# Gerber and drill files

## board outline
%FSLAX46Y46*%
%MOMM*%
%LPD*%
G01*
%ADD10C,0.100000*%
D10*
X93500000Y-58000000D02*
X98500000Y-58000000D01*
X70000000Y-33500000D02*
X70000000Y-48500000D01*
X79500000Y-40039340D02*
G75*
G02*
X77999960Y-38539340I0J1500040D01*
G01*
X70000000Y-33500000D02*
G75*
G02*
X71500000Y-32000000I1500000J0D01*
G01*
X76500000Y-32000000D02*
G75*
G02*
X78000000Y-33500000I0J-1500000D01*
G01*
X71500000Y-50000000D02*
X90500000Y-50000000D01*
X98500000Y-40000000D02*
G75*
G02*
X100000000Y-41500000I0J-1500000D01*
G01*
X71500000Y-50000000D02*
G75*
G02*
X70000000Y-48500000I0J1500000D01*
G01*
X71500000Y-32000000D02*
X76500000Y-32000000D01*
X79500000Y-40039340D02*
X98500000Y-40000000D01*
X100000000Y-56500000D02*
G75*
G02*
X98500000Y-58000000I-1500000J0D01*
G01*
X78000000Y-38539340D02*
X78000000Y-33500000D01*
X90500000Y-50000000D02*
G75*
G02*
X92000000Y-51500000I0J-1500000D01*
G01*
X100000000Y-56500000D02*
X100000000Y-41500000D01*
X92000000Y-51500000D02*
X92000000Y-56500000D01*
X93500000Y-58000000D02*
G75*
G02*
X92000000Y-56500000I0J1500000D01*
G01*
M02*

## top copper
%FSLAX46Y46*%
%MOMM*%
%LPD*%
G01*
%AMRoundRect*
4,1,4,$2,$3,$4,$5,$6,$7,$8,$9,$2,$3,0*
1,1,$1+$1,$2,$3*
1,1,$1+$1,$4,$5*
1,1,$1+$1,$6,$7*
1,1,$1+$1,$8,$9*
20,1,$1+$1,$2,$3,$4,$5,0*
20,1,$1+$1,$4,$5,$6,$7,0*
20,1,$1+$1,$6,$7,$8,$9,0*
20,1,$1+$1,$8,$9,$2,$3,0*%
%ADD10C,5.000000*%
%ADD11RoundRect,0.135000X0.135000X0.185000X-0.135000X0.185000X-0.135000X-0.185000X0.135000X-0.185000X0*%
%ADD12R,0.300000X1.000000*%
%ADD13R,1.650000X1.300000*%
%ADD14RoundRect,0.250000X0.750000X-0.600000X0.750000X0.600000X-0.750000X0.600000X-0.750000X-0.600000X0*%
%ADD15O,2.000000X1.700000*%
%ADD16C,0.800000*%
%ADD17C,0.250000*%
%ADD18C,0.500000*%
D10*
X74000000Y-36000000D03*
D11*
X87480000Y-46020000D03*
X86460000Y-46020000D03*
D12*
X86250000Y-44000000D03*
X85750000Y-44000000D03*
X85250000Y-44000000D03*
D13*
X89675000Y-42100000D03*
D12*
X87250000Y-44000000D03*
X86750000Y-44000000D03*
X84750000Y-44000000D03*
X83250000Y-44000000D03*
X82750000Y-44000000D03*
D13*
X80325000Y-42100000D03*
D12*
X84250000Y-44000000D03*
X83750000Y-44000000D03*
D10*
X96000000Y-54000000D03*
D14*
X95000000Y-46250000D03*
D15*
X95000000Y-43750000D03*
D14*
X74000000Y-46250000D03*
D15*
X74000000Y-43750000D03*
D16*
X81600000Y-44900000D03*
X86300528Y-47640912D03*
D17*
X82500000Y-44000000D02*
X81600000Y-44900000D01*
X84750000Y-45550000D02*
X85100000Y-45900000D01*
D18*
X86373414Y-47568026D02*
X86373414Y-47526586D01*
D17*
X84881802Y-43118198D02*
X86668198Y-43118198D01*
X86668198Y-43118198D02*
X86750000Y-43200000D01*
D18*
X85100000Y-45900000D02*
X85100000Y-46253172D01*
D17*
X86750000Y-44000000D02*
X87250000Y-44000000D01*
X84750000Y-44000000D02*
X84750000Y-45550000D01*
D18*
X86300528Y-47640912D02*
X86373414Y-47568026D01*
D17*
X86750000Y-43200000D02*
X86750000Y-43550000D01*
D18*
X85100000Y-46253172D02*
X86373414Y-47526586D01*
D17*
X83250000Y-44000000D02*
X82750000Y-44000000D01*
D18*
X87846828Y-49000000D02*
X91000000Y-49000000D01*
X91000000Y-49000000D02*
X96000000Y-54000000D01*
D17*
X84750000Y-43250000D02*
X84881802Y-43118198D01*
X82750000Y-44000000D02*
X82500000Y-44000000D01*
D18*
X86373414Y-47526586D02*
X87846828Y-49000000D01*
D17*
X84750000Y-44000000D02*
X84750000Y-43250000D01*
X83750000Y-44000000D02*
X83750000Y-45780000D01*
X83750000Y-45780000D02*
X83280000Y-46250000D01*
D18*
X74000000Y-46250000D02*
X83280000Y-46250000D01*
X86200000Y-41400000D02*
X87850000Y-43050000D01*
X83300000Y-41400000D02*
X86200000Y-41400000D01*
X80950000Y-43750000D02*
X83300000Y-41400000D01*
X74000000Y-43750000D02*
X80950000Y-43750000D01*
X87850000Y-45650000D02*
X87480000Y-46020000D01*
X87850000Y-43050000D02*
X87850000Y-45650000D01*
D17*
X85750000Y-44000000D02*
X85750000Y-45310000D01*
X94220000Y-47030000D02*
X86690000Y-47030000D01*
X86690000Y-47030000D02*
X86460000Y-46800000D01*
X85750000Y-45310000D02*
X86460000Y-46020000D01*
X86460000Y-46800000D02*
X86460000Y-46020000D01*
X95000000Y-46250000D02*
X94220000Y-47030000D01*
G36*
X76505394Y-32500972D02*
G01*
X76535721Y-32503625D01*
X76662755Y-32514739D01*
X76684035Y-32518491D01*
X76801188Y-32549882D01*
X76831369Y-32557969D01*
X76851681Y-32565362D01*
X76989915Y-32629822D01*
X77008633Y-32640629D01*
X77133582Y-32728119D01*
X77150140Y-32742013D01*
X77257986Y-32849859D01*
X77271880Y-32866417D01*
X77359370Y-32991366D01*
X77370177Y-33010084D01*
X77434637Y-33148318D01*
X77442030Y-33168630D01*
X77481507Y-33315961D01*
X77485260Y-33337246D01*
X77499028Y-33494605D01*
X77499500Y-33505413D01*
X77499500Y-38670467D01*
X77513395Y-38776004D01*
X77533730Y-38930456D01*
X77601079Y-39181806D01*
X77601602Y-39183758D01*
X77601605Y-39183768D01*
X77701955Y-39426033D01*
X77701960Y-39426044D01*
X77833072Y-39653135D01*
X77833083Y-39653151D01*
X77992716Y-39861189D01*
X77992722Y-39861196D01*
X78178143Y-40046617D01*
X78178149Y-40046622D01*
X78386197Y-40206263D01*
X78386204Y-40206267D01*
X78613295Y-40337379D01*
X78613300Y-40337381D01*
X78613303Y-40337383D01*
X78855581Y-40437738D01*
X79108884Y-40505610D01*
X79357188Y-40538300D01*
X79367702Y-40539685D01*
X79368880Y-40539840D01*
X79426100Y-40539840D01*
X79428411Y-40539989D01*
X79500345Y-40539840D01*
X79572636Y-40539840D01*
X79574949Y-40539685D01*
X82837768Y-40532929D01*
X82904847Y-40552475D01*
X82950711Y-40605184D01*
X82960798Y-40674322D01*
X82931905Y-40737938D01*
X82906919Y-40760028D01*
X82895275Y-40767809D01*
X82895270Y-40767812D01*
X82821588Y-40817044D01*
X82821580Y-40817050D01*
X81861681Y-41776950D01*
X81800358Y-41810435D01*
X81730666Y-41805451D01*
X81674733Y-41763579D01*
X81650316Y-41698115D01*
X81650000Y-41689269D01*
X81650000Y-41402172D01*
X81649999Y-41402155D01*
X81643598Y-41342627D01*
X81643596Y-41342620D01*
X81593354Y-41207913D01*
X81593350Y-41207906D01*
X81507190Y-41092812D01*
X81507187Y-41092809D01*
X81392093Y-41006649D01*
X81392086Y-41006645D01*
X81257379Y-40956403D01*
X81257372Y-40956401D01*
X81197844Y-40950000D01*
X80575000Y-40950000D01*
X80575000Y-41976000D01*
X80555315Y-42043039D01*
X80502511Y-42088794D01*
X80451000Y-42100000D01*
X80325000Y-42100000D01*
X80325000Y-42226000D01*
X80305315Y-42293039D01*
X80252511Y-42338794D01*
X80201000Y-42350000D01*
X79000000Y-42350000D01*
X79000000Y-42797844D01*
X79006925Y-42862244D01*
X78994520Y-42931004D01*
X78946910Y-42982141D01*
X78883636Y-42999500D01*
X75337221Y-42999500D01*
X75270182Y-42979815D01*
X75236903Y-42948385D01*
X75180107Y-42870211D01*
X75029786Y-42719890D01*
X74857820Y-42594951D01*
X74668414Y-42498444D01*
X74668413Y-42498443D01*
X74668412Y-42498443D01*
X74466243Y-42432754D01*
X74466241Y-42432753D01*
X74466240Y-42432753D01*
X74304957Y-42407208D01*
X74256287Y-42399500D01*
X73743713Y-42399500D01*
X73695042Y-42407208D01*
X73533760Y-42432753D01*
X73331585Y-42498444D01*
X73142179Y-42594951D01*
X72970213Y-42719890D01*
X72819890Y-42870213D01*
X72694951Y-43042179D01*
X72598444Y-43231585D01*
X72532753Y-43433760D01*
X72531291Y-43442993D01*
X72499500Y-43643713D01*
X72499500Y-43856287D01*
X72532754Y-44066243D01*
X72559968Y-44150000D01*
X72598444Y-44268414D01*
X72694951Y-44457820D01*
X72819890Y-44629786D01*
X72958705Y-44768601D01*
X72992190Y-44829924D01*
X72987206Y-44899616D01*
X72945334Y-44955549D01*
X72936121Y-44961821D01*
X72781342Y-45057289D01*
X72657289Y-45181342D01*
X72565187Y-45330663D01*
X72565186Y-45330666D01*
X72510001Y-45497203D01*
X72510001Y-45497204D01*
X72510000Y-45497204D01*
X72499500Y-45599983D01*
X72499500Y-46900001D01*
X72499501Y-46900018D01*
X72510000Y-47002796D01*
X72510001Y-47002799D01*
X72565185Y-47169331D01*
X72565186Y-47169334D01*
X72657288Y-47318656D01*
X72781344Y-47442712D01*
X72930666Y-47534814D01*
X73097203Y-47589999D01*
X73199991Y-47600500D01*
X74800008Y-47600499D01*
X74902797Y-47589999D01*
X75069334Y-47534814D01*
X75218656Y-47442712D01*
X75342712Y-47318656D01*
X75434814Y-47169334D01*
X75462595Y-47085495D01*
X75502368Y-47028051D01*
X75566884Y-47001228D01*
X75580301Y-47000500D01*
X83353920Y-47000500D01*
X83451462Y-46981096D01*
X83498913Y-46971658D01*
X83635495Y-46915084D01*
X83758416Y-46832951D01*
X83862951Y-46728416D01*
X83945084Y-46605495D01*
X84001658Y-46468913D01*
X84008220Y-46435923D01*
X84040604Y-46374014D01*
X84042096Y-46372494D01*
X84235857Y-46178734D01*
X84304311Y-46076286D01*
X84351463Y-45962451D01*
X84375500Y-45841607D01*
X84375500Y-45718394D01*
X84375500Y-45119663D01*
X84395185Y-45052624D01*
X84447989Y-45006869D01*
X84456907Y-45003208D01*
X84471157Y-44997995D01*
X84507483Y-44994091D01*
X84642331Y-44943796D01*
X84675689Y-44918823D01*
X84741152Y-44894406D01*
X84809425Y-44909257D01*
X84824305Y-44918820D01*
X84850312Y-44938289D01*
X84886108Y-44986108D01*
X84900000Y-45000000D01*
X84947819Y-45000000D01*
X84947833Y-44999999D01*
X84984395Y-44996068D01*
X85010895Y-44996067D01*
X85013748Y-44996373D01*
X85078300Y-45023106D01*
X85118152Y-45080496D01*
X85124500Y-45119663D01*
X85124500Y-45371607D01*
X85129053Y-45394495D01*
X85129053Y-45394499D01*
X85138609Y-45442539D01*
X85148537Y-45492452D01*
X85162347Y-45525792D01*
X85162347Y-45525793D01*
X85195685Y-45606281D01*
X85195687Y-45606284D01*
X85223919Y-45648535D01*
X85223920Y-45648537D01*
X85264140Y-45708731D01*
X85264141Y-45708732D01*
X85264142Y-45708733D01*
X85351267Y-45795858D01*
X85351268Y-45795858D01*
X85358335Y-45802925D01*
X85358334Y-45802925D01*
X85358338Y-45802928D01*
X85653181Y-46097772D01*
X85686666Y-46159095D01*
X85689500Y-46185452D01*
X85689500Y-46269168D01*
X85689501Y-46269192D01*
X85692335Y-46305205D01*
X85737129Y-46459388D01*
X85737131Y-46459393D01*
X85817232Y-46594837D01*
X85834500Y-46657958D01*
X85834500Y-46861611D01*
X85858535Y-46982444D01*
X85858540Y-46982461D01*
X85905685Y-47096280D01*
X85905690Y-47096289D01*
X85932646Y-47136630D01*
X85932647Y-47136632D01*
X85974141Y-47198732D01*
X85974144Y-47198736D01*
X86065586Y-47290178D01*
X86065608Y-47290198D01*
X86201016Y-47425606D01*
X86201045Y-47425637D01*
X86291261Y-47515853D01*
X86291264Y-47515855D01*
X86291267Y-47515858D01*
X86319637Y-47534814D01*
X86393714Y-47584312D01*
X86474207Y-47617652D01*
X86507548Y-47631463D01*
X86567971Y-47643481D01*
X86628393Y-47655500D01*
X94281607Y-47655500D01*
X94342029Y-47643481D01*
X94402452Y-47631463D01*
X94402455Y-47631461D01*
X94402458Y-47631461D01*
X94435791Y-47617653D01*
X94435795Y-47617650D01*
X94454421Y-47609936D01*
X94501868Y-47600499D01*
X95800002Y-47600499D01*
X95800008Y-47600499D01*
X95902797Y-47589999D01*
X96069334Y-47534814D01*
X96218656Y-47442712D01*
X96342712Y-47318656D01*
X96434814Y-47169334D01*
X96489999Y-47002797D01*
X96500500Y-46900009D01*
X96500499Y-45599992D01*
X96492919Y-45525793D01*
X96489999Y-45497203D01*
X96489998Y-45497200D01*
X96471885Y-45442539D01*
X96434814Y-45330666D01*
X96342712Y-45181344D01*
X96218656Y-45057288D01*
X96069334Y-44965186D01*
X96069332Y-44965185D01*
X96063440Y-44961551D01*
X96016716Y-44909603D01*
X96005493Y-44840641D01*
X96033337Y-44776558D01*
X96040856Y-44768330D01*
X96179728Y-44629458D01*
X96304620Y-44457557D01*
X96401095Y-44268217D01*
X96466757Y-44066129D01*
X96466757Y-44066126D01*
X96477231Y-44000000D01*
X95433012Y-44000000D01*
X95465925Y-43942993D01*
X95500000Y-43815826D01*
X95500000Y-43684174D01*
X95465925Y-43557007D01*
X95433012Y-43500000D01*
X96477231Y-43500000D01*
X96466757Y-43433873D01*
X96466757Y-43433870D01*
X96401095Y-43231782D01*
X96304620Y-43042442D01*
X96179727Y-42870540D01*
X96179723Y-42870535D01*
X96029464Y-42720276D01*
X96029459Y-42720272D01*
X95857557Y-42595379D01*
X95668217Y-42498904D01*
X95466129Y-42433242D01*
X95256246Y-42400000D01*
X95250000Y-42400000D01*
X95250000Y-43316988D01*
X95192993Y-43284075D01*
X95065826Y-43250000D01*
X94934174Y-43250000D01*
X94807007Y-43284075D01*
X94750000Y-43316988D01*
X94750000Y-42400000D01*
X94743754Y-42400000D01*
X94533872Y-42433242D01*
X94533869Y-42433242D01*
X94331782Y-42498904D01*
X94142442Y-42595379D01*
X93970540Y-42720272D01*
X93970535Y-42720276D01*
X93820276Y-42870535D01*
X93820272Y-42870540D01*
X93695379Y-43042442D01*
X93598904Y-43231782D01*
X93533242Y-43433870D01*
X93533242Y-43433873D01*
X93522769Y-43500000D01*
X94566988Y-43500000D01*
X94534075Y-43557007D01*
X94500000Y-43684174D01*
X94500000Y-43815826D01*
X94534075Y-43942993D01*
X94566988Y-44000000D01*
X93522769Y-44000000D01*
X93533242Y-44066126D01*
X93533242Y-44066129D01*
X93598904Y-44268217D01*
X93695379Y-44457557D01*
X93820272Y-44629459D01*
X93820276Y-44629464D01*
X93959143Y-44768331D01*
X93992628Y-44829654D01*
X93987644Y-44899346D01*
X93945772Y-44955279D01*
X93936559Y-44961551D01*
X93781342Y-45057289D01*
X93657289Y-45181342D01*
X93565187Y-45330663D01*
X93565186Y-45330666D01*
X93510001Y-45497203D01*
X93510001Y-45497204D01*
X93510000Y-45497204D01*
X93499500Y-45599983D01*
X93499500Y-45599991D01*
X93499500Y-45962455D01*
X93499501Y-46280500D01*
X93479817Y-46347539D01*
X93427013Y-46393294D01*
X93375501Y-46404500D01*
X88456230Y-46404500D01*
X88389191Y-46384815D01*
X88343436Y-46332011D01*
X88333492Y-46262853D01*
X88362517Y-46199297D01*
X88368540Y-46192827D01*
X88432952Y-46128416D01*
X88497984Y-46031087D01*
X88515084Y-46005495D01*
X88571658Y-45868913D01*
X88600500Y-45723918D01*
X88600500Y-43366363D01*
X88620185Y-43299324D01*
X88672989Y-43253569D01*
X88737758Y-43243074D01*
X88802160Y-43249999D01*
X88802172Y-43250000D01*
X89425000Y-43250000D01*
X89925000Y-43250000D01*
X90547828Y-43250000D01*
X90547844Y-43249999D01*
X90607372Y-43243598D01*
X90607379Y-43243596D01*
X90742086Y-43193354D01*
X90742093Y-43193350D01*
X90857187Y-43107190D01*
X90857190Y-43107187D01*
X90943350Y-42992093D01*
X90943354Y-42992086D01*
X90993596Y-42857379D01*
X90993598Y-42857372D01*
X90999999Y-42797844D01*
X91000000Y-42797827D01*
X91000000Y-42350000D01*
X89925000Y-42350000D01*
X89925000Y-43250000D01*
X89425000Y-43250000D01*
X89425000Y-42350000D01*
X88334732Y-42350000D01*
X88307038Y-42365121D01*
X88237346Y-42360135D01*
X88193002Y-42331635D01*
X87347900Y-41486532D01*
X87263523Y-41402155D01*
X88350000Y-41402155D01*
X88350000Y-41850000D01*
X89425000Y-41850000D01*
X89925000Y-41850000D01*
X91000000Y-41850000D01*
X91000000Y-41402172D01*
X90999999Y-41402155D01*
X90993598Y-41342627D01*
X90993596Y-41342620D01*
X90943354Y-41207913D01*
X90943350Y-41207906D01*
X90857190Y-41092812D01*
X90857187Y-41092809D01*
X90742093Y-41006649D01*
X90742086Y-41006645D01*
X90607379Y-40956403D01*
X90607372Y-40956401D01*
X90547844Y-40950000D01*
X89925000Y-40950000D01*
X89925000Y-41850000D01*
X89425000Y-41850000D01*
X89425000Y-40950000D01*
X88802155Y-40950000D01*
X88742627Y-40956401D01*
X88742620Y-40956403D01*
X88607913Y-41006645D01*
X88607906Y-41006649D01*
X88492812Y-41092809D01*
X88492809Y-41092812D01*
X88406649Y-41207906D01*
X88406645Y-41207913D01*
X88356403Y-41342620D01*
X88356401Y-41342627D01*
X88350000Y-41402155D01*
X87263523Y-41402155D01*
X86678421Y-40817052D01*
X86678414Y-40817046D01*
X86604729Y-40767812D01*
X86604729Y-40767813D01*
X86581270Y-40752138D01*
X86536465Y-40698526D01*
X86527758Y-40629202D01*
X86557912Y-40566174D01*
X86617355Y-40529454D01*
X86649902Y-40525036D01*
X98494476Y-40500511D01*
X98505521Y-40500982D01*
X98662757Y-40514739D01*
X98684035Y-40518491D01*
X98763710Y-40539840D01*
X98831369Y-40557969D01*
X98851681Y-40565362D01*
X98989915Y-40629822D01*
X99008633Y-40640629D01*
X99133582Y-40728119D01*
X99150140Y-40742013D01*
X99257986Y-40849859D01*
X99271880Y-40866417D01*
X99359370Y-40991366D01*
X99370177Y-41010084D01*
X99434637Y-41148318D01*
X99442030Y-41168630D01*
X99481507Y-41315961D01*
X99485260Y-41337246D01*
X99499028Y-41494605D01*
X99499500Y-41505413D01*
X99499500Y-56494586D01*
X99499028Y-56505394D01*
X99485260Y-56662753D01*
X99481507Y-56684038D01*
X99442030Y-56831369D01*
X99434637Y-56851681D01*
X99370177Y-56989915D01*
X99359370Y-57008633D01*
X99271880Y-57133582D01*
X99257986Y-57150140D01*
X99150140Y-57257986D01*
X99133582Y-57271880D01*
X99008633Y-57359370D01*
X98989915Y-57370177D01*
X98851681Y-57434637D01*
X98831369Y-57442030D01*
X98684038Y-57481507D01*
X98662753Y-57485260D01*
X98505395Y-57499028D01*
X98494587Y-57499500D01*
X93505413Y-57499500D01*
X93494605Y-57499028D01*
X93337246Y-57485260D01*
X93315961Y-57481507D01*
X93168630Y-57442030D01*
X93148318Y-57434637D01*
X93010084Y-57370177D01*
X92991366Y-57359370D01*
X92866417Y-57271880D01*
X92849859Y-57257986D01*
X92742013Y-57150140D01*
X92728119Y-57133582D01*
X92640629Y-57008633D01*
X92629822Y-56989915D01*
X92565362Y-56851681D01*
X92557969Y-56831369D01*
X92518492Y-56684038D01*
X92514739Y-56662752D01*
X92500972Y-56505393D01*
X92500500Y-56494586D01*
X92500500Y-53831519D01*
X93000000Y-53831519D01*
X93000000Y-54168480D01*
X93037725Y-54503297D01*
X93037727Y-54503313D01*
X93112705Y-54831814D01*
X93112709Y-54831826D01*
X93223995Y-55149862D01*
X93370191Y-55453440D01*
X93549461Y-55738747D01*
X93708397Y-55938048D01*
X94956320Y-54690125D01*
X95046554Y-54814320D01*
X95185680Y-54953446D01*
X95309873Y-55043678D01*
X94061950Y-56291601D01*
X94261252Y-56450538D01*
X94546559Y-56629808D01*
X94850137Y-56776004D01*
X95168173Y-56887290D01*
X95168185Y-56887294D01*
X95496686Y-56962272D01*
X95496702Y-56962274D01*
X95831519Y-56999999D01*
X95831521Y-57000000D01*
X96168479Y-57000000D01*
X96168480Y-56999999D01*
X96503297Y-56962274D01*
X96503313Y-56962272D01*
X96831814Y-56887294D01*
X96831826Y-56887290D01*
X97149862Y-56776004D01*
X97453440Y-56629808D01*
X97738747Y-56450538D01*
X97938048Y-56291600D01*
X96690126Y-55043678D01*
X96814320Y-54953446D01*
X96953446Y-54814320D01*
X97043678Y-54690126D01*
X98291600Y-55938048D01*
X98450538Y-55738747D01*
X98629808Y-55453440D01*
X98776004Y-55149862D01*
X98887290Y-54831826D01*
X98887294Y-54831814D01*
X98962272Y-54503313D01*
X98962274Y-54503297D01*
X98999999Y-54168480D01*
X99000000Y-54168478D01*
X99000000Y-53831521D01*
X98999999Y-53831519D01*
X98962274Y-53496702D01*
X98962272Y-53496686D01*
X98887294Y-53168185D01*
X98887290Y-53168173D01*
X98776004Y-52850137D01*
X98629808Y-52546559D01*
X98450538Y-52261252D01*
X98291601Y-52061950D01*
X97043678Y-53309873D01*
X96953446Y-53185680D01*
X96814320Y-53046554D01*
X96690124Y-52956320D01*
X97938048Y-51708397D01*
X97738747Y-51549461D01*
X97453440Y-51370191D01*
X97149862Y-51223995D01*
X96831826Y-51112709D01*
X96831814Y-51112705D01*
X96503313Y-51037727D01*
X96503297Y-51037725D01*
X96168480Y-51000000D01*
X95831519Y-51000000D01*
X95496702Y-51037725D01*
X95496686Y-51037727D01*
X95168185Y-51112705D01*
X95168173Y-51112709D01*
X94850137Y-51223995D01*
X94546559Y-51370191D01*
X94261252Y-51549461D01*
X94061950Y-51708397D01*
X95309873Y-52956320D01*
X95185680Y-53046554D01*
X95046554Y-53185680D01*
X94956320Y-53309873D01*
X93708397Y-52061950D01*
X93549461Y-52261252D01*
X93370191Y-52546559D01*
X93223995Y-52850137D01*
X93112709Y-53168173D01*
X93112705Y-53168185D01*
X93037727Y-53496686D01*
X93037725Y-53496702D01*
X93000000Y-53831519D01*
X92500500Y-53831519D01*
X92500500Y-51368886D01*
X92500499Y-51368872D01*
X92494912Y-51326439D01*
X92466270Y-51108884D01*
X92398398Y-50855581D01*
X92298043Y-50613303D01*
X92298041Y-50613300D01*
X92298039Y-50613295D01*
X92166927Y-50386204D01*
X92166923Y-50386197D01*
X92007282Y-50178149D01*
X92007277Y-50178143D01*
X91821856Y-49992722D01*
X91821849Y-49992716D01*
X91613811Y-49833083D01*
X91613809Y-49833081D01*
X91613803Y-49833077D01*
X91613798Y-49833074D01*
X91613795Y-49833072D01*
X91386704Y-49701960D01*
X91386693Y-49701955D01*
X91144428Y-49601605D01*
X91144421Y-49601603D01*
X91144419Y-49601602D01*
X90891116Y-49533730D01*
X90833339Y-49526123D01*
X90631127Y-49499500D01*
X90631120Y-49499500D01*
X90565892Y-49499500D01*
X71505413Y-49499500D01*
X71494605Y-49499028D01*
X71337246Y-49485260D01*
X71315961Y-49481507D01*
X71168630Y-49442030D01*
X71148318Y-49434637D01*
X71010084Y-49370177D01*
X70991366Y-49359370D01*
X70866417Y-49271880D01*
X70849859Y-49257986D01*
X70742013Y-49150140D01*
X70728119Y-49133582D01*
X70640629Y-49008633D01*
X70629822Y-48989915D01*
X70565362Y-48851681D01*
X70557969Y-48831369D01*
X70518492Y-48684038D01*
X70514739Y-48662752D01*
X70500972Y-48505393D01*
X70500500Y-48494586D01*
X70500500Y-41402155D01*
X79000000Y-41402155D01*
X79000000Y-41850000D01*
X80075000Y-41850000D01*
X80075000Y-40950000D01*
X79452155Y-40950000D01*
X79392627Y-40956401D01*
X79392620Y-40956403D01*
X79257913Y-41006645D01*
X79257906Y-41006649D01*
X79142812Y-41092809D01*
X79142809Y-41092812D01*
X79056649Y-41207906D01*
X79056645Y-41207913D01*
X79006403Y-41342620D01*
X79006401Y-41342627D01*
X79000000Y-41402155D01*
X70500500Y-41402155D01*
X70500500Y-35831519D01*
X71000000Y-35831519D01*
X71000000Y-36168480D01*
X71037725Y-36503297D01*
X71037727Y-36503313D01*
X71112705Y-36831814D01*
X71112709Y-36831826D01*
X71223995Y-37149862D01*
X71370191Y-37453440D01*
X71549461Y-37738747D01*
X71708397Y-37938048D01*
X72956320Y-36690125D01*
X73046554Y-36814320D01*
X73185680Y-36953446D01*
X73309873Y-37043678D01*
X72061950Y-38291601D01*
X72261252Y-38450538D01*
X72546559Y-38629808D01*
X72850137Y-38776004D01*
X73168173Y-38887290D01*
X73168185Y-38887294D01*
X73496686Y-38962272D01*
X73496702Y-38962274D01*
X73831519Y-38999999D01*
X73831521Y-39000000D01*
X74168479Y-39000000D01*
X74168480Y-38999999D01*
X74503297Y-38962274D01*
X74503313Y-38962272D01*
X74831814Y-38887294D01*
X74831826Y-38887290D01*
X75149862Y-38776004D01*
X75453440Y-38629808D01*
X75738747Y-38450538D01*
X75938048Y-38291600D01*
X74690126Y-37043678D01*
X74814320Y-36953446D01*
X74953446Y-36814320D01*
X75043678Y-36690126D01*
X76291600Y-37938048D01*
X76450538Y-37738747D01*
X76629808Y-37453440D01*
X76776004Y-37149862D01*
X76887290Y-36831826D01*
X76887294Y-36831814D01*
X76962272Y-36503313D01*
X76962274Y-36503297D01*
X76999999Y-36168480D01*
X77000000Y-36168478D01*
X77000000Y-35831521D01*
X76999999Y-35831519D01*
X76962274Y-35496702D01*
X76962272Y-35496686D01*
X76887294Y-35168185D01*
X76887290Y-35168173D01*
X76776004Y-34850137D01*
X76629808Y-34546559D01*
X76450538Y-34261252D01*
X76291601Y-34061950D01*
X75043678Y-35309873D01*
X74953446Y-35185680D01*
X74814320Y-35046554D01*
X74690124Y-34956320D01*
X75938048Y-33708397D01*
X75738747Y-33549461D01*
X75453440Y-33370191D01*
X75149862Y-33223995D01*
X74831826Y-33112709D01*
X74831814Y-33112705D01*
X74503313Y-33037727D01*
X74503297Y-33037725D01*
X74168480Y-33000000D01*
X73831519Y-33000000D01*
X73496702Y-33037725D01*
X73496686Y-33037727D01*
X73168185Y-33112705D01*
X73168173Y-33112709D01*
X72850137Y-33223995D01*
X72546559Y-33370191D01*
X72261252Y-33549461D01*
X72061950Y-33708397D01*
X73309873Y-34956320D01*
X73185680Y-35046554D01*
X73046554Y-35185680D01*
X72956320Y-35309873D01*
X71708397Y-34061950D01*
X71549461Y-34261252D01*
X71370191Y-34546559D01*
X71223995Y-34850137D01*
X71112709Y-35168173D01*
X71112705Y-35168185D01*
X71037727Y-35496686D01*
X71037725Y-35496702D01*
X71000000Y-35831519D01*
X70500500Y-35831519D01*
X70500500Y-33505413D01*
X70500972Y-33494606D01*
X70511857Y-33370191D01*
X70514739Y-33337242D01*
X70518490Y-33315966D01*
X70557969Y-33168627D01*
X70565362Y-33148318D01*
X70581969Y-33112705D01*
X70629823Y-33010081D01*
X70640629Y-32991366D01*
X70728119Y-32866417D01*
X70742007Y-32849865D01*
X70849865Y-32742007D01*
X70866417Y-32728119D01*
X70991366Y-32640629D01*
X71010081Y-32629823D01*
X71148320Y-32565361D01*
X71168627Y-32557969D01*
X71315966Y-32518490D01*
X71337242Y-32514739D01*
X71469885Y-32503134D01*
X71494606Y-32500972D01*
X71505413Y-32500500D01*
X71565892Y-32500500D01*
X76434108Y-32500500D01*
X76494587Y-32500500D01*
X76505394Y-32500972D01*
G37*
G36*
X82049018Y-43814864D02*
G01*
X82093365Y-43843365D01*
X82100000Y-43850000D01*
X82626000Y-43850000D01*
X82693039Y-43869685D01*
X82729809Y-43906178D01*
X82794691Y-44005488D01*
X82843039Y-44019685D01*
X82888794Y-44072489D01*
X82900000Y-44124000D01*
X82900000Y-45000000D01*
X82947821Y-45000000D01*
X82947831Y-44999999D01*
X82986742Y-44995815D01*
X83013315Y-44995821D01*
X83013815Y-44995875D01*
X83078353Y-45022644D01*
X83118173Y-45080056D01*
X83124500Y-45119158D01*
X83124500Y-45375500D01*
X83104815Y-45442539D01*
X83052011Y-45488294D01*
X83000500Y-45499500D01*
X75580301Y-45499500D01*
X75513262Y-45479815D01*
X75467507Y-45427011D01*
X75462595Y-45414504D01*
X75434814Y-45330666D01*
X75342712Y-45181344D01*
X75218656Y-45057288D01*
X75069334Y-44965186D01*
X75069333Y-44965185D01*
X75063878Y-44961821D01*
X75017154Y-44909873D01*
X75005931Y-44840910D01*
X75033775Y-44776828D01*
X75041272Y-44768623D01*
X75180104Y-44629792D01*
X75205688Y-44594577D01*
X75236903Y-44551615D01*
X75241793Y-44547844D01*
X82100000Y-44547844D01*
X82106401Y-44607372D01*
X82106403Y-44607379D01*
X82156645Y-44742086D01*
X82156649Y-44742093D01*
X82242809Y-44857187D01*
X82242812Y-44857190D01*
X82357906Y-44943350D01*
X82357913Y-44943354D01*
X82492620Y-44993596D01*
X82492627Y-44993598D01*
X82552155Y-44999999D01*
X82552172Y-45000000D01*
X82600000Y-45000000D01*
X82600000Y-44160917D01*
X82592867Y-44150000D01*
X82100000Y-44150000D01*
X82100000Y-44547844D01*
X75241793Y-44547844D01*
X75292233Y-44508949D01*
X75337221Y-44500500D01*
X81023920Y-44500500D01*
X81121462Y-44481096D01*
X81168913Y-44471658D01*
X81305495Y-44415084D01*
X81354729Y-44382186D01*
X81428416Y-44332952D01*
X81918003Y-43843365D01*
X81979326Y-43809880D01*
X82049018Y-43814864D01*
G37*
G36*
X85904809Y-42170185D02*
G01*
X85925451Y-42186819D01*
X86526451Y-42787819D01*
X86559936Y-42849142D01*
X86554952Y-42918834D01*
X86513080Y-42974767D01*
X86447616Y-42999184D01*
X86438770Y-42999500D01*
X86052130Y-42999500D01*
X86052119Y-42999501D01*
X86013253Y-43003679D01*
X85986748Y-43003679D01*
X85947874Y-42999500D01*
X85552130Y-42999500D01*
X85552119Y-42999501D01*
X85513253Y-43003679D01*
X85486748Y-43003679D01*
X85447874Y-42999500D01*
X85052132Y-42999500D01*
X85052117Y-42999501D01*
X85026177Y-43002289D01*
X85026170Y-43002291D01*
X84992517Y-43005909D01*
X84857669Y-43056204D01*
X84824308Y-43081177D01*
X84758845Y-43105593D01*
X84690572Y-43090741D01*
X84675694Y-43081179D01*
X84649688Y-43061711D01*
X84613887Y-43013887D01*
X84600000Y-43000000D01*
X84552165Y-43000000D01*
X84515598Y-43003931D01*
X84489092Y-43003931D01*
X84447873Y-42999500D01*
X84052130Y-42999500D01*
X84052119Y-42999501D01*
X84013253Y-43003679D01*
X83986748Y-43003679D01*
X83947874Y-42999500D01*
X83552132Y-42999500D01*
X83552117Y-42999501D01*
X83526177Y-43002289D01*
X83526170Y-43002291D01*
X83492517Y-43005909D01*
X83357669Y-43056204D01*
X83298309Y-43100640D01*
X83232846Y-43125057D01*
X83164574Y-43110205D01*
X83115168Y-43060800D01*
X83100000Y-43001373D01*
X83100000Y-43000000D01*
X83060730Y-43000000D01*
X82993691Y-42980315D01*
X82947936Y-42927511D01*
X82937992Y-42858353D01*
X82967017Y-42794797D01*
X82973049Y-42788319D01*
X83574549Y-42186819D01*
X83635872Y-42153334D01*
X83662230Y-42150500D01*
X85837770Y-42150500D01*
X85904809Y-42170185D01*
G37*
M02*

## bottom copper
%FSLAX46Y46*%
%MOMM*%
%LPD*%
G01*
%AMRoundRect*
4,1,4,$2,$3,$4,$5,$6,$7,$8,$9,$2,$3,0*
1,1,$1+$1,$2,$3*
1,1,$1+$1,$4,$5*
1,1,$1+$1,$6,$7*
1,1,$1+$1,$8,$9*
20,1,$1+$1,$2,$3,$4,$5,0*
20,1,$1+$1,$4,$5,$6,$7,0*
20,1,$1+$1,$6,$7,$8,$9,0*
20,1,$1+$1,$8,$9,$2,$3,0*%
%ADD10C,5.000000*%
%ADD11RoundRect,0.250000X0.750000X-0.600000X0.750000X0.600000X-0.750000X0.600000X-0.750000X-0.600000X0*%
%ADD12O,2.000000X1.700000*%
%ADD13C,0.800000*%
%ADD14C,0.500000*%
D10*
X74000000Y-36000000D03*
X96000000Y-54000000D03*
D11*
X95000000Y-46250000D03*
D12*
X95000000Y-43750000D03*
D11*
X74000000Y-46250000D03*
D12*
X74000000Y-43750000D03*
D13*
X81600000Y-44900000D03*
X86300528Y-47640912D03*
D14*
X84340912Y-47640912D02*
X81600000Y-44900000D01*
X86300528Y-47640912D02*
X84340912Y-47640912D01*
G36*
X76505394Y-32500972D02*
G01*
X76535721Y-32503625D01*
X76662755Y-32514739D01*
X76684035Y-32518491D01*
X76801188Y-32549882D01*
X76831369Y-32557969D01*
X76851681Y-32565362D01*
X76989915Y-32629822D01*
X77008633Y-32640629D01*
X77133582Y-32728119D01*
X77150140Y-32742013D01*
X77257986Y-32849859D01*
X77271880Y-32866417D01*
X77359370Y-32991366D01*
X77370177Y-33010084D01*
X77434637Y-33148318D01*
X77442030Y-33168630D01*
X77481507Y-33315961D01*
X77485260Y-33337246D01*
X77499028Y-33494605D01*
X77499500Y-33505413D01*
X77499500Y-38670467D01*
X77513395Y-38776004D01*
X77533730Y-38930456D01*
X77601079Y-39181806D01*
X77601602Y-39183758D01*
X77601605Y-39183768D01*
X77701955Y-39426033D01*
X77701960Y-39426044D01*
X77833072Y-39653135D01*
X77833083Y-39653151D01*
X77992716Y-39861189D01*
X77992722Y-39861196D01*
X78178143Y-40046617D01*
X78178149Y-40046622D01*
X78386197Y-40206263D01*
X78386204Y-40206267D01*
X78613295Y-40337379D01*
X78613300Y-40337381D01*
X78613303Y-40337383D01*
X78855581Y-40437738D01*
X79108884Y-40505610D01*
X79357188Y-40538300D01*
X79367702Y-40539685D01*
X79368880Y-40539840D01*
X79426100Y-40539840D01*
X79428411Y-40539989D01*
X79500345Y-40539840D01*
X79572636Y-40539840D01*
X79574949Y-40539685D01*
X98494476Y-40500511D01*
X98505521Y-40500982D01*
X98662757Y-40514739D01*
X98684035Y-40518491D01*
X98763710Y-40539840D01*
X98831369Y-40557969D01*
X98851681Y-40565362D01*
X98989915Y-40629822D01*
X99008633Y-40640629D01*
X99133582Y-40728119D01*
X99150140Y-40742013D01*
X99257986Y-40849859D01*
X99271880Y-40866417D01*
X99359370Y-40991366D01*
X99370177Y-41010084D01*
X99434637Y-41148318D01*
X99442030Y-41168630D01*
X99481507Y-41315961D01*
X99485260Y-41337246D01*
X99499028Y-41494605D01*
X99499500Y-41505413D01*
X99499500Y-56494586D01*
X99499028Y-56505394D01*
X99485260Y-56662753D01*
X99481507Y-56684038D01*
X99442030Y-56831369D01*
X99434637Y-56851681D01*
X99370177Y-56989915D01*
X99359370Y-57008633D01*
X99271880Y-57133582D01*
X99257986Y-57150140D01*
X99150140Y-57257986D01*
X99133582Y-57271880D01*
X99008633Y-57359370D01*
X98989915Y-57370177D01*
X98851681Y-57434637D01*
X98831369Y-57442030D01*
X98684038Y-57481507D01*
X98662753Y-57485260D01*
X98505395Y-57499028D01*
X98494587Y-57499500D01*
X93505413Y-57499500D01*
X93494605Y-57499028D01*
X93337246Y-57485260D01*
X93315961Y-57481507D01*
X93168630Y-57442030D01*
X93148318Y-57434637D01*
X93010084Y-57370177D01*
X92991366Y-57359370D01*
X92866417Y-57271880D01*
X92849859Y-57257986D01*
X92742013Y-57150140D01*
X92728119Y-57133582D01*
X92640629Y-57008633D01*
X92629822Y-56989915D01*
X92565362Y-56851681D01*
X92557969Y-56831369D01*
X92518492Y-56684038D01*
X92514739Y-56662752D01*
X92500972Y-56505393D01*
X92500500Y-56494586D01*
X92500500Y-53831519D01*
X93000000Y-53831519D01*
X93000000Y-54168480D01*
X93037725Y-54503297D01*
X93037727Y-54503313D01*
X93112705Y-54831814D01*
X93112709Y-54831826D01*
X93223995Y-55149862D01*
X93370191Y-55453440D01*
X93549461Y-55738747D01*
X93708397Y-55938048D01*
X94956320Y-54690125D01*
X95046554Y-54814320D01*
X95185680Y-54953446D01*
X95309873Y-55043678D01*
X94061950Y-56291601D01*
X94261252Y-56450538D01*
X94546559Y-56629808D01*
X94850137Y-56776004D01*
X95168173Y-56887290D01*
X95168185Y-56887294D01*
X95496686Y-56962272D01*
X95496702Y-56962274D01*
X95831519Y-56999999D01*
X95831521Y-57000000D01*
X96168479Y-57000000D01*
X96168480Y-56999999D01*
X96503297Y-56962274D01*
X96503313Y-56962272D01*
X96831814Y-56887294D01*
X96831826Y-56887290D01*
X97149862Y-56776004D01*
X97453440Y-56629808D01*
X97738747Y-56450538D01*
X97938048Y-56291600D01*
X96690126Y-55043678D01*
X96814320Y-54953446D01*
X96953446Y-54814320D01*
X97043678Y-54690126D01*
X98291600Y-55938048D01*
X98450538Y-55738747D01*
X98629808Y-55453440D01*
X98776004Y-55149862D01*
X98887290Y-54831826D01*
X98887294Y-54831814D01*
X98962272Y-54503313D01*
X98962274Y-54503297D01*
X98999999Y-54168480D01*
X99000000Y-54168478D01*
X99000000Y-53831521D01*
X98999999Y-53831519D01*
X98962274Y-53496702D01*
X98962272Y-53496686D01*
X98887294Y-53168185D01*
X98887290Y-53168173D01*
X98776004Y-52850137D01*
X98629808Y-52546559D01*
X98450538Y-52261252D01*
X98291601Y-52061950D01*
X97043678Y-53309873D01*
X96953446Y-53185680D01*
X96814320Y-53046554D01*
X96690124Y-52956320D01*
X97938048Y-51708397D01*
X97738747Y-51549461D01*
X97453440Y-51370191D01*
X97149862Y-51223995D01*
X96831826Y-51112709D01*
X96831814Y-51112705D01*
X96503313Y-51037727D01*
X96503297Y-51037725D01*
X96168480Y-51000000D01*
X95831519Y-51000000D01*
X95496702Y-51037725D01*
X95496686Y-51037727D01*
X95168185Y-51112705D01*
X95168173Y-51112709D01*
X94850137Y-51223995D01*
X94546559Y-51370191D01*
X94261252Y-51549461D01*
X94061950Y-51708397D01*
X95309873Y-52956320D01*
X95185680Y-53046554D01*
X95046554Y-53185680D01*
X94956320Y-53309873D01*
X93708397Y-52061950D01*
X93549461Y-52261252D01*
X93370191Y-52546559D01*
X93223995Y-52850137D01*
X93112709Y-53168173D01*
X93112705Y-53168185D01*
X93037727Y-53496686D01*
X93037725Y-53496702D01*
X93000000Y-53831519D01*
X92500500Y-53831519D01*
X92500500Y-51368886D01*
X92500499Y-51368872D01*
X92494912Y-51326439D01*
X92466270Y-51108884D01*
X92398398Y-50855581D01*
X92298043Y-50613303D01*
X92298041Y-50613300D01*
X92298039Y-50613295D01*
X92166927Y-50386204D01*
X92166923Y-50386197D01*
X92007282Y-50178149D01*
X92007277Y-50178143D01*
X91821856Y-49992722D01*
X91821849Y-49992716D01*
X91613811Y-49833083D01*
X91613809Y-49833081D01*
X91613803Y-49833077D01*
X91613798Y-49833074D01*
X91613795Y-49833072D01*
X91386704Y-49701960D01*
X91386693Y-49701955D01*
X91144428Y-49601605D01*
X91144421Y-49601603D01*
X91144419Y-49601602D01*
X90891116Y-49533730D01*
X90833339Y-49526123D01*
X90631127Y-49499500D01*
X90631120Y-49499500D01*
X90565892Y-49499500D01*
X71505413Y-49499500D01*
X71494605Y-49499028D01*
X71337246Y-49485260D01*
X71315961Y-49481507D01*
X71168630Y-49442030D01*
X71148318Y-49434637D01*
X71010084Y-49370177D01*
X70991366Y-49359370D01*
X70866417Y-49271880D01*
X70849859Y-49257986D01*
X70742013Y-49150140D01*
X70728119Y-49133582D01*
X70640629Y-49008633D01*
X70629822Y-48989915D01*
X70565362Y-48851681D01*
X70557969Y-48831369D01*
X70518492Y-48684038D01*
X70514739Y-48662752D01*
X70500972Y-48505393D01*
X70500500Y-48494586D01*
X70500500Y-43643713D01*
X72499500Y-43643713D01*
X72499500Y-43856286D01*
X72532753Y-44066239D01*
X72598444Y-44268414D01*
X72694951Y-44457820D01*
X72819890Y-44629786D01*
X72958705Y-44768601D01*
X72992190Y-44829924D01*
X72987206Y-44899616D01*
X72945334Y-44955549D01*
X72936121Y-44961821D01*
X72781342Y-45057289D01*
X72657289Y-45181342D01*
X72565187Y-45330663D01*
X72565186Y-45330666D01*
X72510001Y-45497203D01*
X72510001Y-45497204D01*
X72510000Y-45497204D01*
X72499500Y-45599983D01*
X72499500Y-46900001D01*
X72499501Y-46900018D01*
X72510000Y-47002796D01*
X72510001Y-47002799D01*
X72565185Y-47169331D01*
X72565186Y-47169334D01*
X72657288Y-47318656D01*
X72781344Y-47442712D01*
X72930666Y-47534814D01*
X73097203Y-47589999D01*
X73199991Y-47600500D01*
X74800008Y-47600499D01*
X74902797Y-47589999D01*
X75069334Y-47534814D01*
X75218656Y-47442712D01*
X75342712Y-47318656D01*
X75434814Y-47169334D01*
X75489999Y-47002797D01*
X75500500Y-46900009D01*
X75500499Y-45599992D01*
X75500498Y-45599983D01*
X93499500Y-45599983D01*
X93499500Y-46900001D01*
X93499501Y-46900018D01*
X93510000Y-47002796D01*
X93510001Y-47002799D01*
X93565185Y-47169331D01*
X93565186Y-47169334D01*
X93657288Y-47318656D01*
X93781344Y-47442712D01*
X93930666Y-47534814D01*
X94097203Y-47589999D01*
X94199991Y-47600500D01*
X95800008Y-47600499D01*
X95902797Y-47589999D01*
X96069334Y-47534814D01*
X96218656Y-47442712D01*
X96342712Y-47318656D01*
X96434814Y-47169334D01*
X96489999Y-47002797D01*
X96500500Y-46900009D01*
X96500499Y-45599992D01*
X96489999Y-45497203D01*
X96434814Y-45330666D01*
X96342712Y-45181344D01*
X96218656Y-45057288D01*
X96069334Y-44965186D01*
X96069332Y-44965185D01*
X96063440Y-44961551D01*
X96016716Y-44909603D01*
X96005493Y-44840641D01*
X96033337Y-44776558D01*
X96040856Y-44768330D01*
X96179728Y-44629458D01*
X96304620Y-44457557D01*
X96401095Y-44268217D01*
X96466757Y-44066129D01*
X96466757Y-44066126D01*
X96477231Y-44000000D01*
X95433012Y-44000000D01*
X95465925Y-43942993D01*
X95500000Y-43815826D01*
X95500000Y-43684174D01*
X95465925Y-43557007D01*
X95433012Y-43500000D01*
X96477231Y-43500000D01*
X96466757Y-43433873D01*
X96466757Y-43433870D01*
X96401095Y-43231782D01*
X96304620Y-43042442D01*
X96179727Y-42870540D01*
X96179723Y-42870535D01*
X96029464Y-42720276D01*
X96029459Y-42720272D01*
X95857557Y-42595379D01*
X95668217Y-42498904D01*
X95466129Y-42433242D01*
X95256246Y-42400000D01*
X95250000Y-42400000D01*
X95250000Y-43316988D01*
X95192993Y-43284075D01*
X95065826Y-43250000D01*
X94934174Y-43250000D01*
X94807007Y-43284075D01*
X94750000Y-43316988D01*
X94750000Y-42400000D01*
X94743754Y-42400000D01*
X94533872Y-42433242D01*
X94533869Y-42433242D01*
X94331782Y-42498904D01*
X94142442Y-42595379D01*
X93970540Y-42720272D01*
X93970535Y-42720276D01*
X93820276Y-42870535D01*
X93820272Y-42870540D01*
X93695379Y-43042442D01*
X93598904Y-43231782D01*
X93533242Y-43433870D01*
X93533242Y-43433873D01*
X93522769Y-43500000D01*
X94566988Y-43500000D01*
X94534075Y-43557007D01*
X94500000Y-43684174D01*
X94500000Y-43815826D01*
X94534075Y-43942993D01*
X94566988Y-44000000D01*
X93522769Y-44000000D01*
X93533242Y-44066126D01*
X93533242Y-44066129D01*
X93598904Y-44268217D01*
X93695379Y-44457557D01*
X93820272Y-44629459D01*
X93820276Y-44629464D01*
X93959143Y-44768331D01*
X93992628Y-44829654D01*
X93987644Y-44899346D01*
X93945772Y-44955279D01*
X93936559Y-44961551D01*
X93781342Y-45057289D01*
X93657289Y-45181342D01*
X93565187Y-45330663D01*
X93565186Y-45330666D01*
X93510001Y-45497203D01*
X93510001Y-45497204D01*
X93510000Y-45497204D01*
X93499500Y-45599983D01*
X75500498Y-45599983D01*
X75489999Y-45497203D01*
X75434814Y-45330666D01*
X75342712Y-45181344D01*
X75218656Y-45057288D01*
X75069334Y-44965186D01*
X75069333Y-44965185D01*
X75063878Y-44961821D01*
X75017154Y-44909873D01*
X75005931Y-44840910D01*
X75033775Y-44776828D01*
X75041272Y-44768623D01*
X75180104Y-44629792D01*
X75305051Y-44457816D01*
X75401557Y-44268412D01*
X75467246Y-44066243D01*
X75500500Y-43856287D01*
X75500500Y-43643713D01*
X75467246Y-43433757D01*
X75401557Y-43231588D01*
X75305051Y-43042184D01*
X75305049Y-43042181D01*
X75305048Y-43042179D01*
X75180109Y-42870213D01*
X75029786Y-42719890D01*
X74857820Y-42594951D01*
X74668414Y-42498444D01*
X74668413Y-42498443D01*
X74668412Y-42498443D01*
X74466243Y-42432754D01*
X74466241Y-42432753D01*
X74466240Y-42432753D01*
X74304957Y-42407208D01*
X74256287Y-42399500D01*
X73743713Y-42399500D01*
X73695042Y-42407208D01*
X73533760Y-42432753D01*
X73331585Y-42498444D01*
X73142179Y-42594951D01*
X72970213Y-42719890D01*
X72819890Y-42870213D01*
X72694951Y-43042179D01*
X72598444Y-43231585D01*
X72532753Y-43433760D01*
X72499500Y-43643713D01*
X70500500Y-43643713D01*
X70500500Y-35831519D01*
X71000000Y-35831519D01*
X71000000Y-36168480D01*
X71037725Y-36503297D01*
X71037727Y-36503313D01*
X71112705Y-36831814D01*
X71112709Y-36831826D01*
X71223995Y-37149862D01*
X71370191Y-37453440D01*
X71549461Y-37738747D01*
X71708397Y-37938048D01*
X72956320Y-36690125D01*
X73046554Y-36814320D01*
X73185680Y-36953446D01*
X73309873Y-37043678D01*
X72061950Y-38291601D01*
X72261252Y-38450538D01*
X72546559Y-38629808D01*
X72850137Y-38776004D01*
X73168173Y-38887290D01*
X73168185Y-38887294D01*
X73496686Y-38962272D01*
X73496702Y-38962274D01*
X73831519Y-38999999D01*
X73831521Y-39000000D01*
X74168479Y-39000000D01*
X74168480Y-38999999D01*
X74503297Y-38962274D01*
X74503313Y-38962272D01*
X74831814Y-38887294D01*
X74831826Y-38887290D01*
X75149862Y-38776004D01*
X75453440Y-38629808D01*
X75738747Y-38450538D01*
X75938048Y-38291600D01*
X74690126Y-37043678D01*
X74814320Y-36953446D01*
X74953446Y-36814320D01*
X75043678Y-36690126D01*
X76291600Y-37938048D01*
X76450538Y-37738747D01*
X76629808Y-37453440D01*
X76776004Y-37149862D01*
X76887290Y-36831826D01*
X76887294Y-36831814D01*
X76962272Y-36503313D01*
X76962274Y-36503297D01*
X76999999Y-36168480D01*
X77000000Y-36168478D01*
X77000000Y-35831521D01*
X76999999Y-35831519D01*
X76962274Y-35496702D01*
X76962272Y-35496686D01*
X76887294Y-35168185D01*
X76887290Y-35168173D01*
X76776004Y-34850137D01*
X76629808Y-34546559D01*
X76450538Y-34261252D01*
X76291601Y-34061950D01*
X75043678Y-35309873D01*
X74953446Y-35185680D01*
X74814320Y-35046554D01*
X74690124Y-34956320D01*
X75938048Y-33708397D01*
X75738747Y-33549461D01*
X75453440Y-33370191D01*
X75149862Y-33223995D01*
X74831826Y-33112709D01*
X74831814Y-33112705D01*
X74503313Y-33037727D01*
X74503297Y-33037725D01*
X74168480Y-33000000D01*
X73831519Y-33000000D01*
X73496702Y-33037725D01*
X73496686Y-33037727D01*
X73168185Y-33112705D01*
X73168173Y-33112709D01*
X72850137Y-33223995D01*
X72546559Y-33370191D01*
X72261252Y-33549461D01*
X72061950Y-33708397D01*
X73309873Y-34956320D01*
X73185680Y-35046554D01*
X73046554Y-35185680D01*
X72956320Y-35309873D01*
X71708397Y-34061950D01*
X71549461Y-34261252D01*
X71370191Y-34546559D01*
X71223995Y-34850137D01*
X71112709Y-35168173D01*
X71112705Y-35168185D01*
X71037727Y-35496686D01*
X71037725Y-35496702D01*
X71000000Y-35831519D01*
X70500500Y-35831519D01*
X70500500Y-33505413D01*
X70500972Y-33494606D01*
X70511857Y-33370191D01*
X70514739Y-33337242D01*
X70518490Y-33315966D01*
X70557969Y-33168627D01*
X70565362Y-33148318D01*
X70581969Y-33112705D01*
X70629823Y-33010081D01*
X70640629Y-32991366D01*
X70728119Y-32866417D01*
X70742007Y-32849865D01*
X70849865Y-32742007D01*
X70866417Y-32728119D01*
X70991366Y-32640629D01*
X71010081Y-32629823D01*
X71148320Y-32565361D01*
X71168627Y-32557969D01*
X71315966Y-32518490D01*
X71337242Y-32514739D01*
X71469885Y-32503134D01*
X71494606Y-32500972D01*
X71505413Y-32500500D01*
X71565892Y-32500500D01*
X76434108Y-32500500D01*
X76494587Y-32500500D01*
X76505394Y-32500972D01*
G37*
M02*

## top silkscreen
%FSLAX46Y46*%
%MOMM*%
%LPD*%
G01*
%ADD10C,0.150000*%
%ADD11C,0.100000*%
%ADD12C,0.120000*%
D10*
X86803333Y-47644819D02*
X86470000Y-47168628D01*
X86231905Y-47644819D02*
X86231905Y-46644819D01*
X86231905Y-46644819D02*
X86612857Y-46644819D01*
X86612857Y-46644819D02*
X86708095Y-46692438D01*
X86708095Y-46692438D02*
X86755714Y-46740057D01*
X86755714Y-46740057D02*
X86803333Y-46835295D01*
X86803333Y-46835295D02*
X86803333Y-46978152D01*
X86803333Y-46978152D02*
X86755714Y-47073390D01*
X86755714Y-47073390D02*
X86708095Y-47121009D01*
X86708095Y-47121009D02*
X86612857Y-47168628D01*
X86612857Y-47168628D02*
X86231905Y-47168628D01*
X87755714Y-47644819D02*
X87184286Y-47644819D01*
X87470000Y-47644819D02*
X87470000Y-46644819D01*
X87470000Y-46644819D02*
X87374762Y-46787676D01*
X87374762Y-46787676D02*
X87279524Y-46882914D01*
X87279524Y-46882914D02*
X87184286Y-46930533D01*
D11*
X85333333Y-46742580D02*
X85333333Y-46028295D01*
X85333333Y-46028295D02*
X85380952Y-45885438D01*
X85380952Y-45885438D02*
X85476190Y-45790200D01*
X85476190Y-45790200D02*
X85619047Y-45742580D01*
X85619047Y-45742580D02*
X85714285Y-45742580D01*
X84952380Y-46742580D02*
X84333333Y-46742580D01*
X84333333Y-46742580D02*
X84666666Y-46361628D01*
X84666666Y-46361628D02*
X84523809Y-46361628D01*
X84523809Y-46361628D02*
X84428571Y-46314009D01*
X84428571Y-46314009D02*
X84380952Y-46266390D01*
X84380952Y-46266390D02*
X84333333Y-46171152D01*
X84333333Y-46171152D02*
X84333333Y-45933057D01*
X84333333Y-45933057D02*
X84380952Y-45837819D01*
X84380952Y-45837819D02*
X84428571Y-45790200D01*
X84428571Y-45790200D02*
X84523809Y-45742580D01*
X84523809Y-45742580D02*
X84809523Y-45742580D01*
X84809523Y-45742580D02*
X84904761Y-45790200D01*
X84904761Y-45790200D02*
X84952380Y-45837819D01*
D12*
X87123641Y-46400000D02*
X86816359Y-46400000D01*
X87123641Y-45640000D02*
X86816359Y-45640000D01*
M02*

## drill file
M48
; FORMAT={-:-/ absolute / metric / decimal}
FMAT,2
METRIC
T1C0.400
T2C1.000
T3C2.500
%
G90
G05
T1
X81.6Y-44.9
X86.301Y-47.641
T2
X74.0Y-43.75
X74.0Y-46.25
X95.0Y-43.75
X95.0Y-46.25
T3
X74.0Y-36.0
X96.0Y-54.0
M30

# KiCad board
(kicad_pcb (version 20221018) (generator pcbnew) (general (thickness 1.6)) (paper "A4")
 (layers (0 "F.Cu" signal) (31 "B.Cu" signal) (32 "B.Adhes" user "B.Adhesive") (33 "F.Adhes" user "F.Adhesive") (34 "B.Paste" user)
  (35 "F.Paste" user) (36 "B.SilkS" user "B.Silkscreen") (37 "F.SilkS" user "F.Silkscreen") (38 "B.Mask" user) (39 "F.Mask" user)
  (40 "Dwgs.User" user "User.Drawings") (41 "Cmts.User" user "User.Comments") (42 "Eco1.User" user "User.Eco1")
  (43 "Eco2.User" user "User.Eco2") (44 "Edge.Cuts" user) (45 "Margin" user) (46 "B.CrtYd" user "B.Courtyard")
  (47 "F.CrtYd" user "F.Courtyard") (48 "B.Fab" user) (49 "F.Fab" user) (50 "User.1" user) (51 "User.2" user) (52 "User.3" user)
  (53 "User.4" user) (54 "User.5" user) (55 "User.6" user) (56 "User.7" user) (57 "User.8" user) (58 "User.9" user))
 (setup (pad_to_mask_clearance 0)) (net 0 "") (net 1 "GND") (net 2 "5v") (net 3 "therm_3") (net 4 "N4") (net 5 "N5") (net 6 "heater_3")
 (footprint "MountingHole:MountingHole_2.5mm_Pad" (layer "F.Cu") (at 74 36)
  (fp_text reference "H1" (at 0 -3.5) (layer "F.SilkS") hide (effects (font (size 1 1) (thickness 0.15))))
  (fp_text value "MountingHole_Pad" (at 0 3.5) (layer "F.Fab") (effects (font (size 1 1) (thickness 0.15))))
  (pad "1" thru_hole circle (at 0 0) (size 5 5) (drill 2.5) (layers "*.Cu" "*.Mask") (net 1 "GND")))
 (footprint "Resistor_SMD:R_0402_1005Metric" (layer "F.Cu") (at 86.97 46.02 180)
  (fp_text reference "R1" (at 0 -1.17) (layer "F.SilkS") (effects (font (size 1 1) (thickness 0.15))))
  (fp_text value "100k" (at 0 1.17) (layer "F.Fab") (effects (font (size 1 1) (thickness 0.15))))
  (fp_line (start -0.153641 -0.38) (end 0.153641 -0.38) (stroke (width 0.12) (type solid)) (layer "F.SilkS"))
  (fp_line (start -0.153641 0.38) (end 0.153641 0.38) (stroke (width 0.12) (type solid)) (layer "F.SilkS"))
  (pad "1" smd roundrect (at -0.51 0 180) (size 0.54 0.64) (layers "F.Cu" "F.Paste" "F.Mask") (roundrect_rratio 0.25) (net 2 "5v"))
  (pad "2" smd roundrect (at 0.51 0 180) (size 0.54 0.64) (layers "F.Cu" "F.Paste" "F.Mask") (roundrect_rratio 0.25) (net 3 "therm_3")))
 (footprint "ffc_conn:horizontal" (layer "F.Cu") (at 85 43.5 180)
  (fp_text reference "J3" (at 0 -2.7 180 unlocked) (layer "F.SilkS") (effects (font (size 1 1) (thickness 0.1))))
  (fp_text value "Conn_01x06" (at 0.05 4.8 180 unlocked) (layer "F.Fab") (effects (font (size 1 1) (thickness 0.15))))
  (pad "1" smd rect (at -1.25 -0.5 180) (size 0.3 1) (layers "F.Cu" "F.Paste" "F.Mask") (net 2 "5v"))
  (pad "2" smd rect (at -0.75 -0.5 180) (size 0.3 1) (layers "F.Cu" "F.Paste" "F.Mask") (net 3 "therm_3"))
  (pad "3" smd rect (at -0.25 -0.5 180) (size 0.3 1) (layers "F.Cu" "F.Paste" "F.Mask") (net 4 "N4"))
  (pad "4" smd rect (at -4.675 1.4 180) (size 1.65 1.3) (layers "F.Cu" "F.Paste" "F.Mask") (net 1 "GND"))
  (pad "4" smd rect (at -2.25 -0.5 180) (size 0.3 1) (layers "F.Cu" "F.Paste" "F.Mask") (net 1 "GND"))
  (pad "4" smd rect (at -1.75 -0.5 180) (size 0.3 1) (layers "F.Cu" "F.Paste" "F.Mask") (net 1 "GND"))
  (pad "4" smd rect (at 0.25 -0.5 180) (size 0.3 1) (layers "F.Cu" "F.Paste" "F.Mask") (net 1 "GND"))
  (pad "4" smd rect (at 1.75 -0.5 180) (size 0.3 1) (layers "F.Cu" "F.Paste" "F.Mask") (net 1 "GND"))
  (pad "4" smd rect (at 2.25 -0.5 180) (size 0.3 1) (layers "F.Cu" "F.Paste" "F.Mask") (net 1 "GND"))
  (pad "4" smd rect (at 4.675 1.4 180) (size 1.65 1.3) (layers "F.Cu" "F.Paste" "F.Mask") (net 1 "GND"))
  (pad "5" smd rect (at 0.75 -0.5 180) (size 0.3 1) (layers "F.Cu" "F.Paste" "F.Mask") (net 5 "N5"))
  (pad "6" smd rect (at 1.25 -0.5 180) (size 0.3 1) (layers "F.Cu" "F.Paste" "F.Mask") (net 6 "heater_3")))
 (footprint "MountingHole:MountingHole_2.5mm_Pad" (layer "F.Cu") (at 96 54)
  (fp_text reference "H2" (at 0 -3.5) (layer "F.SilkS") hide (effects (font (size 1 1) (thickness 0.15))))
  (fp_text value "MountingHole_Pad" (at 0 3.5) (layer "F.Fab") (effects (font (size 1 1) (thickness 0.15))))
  (pad "1" thru_hole circle (at 0 0) (size 5 5) (drill 2.5) (layers "*.Cu" "*.Mask") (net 1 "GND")))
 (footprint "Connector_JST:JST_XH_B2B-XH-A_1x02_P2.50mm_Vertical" (layer "B.Cu") (at 95 46.25 90)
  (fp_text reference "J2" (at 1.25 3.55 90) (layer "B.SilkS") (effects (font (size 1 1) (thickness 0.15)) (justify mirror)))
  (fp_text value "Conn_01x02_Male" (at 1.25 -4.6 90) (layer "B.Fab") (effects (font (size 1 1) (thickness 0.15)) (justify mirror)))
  (pad "1" thru_hole roundrect (at 0 0 90) (size 1.7 2) (drill 1) (layers "*.Cu" "*.Mask") (roundrect_rratio 0.147059) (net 3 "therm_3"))
  (pad "2" thru_hole oval (at 2.5 0 90) (size 1.7 2) (drill 1) (layers "*.Cu" "*.Mask") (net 1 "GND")))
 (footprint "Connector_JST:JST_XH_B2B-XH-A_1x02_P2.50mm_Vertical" (layer "B.Cu") (at 74 46.25 90)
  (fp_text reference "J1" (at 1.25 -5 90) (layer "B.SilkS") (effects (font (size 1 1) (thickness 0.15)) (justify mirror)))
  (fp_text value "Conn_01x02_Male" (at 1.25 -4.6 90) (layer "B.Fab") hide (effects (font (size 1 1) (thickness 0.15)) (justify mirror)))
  (pad "1" thru_hole roundrect (at 0 0 90) (size 1.7 2) (drill 1) (layers "*.Cu" "*.Mask") (roundrect_rratio 0.147059) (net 6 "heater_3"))
  (pad "2" thru_hole oval (at 2.5 0 90) (size 1.7 2) (drill 1) (layers "*.Cu" "*.Mask") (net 2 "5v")))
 (gr_line (start 93.5 58) (end 98.5 58) (stroke (width 0.1) (type default)) (layer "Edge.Cuts"))
 (gr_line (start 70 33.5) (end 70 48.5) (stroke (width 0.1) (type default)) (layer "Edge.Cuts"))
 (gr_arc (start 79.5 40.03934) (mid 78.43934 39.6) (end 78 38.53934) (stroke (width 0.1) (type default)) (layer "Edge.Cuts"))
 (gr_arc (start 70 33.5) (mid 70.43934 32.43934) (end 71.5 32) (stroke (width 0.1) (type default)) (layer "Edge.Cuts"))
 (gr_arc (start 76.5 32) (mid 77.56066 32.43934) (end 78 33.5) (stroke (width 0.1) (type default)) (layer "Edge.Cuts"))
 (gr_line (start 71.5 50) (end 90.5 50) (stroke (width 0.1) (type default)) (layer "Edge.Cuts"))
 (gr_arc (start 98.5 40) (mid 99.56066 40.43934) (end 100 41.5) (stroke (width 0.1) (type default)) (layer "Edge.Cuts"))
 (gr_arc (start 71.5 50) (mid 70.43934 49.56066) (end 70 48.5) (stroke (width 0.1) (type default)) (layer "Edge.Cuts"))
 (gr_line (start 71.5 32) (end 76.5 32) (stroke (width 0.1) (type default)) (layer "Edge.Cuts"))
 (gr_line (start 79.5 40.03934) (end 98.5 40) (stroke (width 0.1) (type default)) (layer "Edge.Cuts"))
 (gr_arc (start 100 56.5) (mid 99.56066 57.56066) (end 98.5 58) (stroke (width 0.1) (type default)) (layer "Edge.Cuts"))
 (gr_line (start 78 38.53934) (end 78 33.5) (stroke (width 0.1) (type default)) (layer "Edge.Cuts"))
 (gr_arc (start 90.5 50) (mid 91.56066 50.43934) (end 92 51.5) (stroke (width 0.1) (type default)) (layer "Edge.Cuts"))
 (gr_line (start 100 56.5) (end 100 41.5) (stroke (width 0.1) (type default)) (layer "Edge.Cuts"))
 (gr_line (start 92 51.5) (end 92 56.5) (stroke (width 0.1) (type default)) (layer "Edge.Cuts"))
 (gr_arc (start 93.5 58) (mid 92.43934 57.56066) (end 92 56.5) (stroke (width 0.1) (type default)) (layer "Edge.Cuts"))
 (segment (start 82.5 44) (end 81.6 44.9) (width 0.25) (layer "F.Cu") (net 1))
 (segment (start 84.75 45.55) (end 85.1 45.9) (width 0.25) (layer "F.Cu") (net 1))
 (segment (start 86.373414 47.568026) (end 86.373414 47.526586) (width 0.5) (layer "F.Cu") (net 1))
 (segment (start 84.881802 43.118198) (end 86.668198 43.118198) (width 0.25) (layer "F.Cu") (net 1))
 (segment (start 86.668198 43.118198) (end 86.75 43.2) (width 0.25) (layer "F.Cu") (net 1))
 (segment (start 85.1 45.9) (end 85.1 46.253172) (width 0.5) (layer "F.Cu") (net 1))
 (segment (start 86.75 44) (end 87.25 44) (width 0.25) (layer "F.Cu") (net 1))
 (segment (start 84.75 44) (end 84.75 45.55) (width 0.25) (layer "F.Cu") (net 1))
 (segment (start 86.300528 47.640912) (end 86.373414 47.568026) (width 0.5) (layer "F.Cu") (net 1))
 (segment (start 86.75 43.2) (end 86.75 43.55) (width 0.25) (layer "F.Cu") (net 1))
 (segment (start 85.1 46.253172) (end 86.373414 47.526586) (width 0.5) (layer "F.Cu") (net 1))
 (segment (start 83.25 44) (end 82.75 44) (width 0.25) (layer "F.Cu") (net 1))
 (segment (start 87.846828 49) (end 91 49) (width 0.5) (layer "F.Cu") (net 1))
 (segment (start 91 49) (end 96 54) (width 0.5) (layer "F.Cu") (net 1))
 (segment (start 84.75 43.25) (end 84.881802 43.118198) (width 0.25) (layer "F.Cu") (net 1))
 (segment (start 82.75 44) (end 82.5 44) (width 0.25) (layer "F.Cu") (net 1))
 (segment (start 86.373414 47.526586) (end 87.846828 49) (width 0.5) (layer "F.Cu") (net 1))
 (segment (start 84.75 44) (end 84.75 43.25) (width 0.25) (layer "F.Cu") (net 1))
 (via (at 81.6 44.9) (size 0.8) (drill 0.4) (layers "F.Cu" "B.Cu") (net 1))
 (via (at 86.300528 47.640912) (size 0.8) (drill 0.4) (layers "F.Cu" "B.Cu") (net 1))
 (segment (start 84.340912 47.640912) (end 81.6 44.9) (width 0.5) (layer "B.Cu") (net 1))
 (segment (start 86.300528 47.640912) (end 84.340912 47.640912) (width 0.5) (layer "B.Cu") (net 1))
 (segment (start 83.75 44) (end 83.75 45.78) (width 0.25) (layer "F.Cu") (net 6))
 (segment (start 83.75 45.78) (end 83.28 46.25) (width 0.25) (layer "F.Cu") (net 6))
 (segment (start 74 46.25) (end 83.28 46.25) (width 0.5) (layer "F.Cu") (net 6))
 (segment (start 86.2 41.4) (end 87.85 43.05) (width 0.5) (layer "F.Cu") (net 2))
 (segment (start 83.3 41.4) (end 86.2 41.4) (width 0.5) (layer "F.Cu") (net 2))
 (segment (start 80.95 43.75) (end 83.3 41.4) (width 0.5) (layer "F.Cu") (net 2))
 (segment (start 74 43.75) (end 80.95 43.75) (width 0.5) (layer "F.Cu") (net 2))
 (segment (start 87.85 45.65) (end 87.48 46.02) (width 0.5) (layer "F.Cu") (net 2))
 (segment (start 87.85 43.05) (end 87.85 45.65) (width 0.5) (layer "F.Cu") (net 2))
 (segment (start 85.75 44) (end 85.75 45.31) (width 0.25) (layer "F.Cu") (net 3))
 (segment (start 94.22 47.03) (end 86.69 47.03) (width 0.25) (layer "F.Cu") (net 3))
 (segment (start 86.69 47.03) (end 86.46 46.8) (width 0.25) (layer "F.Cu") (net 3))
 (segment (start 85.75 45.31) (end 86.46 46.02) (width 0.25) (layer "F.Cu") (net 3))
 (segment (start 86.46 46.8) (end 86.46 46.02) (width 0.25) (layer "F.Cu") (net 3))
 (segment (start 95 46.25) (end 94.22 47.03) (width 0.25) (layer "F.Cu") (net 3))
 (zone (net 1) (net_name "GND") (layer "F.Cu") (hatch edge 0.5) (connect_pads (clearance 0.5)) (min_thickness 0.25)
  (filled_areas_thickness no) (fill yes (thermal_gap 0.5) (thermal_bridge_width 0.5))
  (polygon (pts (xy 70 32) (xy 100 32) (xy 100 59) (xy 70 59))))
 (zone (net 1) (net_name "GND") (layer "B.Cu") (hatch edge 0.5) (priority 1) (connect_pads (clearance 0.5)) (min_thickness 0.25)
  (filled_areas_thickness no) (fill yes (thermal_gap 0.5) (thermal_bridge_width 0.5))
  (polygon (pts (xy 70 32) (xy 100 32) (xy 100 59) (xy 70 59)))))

